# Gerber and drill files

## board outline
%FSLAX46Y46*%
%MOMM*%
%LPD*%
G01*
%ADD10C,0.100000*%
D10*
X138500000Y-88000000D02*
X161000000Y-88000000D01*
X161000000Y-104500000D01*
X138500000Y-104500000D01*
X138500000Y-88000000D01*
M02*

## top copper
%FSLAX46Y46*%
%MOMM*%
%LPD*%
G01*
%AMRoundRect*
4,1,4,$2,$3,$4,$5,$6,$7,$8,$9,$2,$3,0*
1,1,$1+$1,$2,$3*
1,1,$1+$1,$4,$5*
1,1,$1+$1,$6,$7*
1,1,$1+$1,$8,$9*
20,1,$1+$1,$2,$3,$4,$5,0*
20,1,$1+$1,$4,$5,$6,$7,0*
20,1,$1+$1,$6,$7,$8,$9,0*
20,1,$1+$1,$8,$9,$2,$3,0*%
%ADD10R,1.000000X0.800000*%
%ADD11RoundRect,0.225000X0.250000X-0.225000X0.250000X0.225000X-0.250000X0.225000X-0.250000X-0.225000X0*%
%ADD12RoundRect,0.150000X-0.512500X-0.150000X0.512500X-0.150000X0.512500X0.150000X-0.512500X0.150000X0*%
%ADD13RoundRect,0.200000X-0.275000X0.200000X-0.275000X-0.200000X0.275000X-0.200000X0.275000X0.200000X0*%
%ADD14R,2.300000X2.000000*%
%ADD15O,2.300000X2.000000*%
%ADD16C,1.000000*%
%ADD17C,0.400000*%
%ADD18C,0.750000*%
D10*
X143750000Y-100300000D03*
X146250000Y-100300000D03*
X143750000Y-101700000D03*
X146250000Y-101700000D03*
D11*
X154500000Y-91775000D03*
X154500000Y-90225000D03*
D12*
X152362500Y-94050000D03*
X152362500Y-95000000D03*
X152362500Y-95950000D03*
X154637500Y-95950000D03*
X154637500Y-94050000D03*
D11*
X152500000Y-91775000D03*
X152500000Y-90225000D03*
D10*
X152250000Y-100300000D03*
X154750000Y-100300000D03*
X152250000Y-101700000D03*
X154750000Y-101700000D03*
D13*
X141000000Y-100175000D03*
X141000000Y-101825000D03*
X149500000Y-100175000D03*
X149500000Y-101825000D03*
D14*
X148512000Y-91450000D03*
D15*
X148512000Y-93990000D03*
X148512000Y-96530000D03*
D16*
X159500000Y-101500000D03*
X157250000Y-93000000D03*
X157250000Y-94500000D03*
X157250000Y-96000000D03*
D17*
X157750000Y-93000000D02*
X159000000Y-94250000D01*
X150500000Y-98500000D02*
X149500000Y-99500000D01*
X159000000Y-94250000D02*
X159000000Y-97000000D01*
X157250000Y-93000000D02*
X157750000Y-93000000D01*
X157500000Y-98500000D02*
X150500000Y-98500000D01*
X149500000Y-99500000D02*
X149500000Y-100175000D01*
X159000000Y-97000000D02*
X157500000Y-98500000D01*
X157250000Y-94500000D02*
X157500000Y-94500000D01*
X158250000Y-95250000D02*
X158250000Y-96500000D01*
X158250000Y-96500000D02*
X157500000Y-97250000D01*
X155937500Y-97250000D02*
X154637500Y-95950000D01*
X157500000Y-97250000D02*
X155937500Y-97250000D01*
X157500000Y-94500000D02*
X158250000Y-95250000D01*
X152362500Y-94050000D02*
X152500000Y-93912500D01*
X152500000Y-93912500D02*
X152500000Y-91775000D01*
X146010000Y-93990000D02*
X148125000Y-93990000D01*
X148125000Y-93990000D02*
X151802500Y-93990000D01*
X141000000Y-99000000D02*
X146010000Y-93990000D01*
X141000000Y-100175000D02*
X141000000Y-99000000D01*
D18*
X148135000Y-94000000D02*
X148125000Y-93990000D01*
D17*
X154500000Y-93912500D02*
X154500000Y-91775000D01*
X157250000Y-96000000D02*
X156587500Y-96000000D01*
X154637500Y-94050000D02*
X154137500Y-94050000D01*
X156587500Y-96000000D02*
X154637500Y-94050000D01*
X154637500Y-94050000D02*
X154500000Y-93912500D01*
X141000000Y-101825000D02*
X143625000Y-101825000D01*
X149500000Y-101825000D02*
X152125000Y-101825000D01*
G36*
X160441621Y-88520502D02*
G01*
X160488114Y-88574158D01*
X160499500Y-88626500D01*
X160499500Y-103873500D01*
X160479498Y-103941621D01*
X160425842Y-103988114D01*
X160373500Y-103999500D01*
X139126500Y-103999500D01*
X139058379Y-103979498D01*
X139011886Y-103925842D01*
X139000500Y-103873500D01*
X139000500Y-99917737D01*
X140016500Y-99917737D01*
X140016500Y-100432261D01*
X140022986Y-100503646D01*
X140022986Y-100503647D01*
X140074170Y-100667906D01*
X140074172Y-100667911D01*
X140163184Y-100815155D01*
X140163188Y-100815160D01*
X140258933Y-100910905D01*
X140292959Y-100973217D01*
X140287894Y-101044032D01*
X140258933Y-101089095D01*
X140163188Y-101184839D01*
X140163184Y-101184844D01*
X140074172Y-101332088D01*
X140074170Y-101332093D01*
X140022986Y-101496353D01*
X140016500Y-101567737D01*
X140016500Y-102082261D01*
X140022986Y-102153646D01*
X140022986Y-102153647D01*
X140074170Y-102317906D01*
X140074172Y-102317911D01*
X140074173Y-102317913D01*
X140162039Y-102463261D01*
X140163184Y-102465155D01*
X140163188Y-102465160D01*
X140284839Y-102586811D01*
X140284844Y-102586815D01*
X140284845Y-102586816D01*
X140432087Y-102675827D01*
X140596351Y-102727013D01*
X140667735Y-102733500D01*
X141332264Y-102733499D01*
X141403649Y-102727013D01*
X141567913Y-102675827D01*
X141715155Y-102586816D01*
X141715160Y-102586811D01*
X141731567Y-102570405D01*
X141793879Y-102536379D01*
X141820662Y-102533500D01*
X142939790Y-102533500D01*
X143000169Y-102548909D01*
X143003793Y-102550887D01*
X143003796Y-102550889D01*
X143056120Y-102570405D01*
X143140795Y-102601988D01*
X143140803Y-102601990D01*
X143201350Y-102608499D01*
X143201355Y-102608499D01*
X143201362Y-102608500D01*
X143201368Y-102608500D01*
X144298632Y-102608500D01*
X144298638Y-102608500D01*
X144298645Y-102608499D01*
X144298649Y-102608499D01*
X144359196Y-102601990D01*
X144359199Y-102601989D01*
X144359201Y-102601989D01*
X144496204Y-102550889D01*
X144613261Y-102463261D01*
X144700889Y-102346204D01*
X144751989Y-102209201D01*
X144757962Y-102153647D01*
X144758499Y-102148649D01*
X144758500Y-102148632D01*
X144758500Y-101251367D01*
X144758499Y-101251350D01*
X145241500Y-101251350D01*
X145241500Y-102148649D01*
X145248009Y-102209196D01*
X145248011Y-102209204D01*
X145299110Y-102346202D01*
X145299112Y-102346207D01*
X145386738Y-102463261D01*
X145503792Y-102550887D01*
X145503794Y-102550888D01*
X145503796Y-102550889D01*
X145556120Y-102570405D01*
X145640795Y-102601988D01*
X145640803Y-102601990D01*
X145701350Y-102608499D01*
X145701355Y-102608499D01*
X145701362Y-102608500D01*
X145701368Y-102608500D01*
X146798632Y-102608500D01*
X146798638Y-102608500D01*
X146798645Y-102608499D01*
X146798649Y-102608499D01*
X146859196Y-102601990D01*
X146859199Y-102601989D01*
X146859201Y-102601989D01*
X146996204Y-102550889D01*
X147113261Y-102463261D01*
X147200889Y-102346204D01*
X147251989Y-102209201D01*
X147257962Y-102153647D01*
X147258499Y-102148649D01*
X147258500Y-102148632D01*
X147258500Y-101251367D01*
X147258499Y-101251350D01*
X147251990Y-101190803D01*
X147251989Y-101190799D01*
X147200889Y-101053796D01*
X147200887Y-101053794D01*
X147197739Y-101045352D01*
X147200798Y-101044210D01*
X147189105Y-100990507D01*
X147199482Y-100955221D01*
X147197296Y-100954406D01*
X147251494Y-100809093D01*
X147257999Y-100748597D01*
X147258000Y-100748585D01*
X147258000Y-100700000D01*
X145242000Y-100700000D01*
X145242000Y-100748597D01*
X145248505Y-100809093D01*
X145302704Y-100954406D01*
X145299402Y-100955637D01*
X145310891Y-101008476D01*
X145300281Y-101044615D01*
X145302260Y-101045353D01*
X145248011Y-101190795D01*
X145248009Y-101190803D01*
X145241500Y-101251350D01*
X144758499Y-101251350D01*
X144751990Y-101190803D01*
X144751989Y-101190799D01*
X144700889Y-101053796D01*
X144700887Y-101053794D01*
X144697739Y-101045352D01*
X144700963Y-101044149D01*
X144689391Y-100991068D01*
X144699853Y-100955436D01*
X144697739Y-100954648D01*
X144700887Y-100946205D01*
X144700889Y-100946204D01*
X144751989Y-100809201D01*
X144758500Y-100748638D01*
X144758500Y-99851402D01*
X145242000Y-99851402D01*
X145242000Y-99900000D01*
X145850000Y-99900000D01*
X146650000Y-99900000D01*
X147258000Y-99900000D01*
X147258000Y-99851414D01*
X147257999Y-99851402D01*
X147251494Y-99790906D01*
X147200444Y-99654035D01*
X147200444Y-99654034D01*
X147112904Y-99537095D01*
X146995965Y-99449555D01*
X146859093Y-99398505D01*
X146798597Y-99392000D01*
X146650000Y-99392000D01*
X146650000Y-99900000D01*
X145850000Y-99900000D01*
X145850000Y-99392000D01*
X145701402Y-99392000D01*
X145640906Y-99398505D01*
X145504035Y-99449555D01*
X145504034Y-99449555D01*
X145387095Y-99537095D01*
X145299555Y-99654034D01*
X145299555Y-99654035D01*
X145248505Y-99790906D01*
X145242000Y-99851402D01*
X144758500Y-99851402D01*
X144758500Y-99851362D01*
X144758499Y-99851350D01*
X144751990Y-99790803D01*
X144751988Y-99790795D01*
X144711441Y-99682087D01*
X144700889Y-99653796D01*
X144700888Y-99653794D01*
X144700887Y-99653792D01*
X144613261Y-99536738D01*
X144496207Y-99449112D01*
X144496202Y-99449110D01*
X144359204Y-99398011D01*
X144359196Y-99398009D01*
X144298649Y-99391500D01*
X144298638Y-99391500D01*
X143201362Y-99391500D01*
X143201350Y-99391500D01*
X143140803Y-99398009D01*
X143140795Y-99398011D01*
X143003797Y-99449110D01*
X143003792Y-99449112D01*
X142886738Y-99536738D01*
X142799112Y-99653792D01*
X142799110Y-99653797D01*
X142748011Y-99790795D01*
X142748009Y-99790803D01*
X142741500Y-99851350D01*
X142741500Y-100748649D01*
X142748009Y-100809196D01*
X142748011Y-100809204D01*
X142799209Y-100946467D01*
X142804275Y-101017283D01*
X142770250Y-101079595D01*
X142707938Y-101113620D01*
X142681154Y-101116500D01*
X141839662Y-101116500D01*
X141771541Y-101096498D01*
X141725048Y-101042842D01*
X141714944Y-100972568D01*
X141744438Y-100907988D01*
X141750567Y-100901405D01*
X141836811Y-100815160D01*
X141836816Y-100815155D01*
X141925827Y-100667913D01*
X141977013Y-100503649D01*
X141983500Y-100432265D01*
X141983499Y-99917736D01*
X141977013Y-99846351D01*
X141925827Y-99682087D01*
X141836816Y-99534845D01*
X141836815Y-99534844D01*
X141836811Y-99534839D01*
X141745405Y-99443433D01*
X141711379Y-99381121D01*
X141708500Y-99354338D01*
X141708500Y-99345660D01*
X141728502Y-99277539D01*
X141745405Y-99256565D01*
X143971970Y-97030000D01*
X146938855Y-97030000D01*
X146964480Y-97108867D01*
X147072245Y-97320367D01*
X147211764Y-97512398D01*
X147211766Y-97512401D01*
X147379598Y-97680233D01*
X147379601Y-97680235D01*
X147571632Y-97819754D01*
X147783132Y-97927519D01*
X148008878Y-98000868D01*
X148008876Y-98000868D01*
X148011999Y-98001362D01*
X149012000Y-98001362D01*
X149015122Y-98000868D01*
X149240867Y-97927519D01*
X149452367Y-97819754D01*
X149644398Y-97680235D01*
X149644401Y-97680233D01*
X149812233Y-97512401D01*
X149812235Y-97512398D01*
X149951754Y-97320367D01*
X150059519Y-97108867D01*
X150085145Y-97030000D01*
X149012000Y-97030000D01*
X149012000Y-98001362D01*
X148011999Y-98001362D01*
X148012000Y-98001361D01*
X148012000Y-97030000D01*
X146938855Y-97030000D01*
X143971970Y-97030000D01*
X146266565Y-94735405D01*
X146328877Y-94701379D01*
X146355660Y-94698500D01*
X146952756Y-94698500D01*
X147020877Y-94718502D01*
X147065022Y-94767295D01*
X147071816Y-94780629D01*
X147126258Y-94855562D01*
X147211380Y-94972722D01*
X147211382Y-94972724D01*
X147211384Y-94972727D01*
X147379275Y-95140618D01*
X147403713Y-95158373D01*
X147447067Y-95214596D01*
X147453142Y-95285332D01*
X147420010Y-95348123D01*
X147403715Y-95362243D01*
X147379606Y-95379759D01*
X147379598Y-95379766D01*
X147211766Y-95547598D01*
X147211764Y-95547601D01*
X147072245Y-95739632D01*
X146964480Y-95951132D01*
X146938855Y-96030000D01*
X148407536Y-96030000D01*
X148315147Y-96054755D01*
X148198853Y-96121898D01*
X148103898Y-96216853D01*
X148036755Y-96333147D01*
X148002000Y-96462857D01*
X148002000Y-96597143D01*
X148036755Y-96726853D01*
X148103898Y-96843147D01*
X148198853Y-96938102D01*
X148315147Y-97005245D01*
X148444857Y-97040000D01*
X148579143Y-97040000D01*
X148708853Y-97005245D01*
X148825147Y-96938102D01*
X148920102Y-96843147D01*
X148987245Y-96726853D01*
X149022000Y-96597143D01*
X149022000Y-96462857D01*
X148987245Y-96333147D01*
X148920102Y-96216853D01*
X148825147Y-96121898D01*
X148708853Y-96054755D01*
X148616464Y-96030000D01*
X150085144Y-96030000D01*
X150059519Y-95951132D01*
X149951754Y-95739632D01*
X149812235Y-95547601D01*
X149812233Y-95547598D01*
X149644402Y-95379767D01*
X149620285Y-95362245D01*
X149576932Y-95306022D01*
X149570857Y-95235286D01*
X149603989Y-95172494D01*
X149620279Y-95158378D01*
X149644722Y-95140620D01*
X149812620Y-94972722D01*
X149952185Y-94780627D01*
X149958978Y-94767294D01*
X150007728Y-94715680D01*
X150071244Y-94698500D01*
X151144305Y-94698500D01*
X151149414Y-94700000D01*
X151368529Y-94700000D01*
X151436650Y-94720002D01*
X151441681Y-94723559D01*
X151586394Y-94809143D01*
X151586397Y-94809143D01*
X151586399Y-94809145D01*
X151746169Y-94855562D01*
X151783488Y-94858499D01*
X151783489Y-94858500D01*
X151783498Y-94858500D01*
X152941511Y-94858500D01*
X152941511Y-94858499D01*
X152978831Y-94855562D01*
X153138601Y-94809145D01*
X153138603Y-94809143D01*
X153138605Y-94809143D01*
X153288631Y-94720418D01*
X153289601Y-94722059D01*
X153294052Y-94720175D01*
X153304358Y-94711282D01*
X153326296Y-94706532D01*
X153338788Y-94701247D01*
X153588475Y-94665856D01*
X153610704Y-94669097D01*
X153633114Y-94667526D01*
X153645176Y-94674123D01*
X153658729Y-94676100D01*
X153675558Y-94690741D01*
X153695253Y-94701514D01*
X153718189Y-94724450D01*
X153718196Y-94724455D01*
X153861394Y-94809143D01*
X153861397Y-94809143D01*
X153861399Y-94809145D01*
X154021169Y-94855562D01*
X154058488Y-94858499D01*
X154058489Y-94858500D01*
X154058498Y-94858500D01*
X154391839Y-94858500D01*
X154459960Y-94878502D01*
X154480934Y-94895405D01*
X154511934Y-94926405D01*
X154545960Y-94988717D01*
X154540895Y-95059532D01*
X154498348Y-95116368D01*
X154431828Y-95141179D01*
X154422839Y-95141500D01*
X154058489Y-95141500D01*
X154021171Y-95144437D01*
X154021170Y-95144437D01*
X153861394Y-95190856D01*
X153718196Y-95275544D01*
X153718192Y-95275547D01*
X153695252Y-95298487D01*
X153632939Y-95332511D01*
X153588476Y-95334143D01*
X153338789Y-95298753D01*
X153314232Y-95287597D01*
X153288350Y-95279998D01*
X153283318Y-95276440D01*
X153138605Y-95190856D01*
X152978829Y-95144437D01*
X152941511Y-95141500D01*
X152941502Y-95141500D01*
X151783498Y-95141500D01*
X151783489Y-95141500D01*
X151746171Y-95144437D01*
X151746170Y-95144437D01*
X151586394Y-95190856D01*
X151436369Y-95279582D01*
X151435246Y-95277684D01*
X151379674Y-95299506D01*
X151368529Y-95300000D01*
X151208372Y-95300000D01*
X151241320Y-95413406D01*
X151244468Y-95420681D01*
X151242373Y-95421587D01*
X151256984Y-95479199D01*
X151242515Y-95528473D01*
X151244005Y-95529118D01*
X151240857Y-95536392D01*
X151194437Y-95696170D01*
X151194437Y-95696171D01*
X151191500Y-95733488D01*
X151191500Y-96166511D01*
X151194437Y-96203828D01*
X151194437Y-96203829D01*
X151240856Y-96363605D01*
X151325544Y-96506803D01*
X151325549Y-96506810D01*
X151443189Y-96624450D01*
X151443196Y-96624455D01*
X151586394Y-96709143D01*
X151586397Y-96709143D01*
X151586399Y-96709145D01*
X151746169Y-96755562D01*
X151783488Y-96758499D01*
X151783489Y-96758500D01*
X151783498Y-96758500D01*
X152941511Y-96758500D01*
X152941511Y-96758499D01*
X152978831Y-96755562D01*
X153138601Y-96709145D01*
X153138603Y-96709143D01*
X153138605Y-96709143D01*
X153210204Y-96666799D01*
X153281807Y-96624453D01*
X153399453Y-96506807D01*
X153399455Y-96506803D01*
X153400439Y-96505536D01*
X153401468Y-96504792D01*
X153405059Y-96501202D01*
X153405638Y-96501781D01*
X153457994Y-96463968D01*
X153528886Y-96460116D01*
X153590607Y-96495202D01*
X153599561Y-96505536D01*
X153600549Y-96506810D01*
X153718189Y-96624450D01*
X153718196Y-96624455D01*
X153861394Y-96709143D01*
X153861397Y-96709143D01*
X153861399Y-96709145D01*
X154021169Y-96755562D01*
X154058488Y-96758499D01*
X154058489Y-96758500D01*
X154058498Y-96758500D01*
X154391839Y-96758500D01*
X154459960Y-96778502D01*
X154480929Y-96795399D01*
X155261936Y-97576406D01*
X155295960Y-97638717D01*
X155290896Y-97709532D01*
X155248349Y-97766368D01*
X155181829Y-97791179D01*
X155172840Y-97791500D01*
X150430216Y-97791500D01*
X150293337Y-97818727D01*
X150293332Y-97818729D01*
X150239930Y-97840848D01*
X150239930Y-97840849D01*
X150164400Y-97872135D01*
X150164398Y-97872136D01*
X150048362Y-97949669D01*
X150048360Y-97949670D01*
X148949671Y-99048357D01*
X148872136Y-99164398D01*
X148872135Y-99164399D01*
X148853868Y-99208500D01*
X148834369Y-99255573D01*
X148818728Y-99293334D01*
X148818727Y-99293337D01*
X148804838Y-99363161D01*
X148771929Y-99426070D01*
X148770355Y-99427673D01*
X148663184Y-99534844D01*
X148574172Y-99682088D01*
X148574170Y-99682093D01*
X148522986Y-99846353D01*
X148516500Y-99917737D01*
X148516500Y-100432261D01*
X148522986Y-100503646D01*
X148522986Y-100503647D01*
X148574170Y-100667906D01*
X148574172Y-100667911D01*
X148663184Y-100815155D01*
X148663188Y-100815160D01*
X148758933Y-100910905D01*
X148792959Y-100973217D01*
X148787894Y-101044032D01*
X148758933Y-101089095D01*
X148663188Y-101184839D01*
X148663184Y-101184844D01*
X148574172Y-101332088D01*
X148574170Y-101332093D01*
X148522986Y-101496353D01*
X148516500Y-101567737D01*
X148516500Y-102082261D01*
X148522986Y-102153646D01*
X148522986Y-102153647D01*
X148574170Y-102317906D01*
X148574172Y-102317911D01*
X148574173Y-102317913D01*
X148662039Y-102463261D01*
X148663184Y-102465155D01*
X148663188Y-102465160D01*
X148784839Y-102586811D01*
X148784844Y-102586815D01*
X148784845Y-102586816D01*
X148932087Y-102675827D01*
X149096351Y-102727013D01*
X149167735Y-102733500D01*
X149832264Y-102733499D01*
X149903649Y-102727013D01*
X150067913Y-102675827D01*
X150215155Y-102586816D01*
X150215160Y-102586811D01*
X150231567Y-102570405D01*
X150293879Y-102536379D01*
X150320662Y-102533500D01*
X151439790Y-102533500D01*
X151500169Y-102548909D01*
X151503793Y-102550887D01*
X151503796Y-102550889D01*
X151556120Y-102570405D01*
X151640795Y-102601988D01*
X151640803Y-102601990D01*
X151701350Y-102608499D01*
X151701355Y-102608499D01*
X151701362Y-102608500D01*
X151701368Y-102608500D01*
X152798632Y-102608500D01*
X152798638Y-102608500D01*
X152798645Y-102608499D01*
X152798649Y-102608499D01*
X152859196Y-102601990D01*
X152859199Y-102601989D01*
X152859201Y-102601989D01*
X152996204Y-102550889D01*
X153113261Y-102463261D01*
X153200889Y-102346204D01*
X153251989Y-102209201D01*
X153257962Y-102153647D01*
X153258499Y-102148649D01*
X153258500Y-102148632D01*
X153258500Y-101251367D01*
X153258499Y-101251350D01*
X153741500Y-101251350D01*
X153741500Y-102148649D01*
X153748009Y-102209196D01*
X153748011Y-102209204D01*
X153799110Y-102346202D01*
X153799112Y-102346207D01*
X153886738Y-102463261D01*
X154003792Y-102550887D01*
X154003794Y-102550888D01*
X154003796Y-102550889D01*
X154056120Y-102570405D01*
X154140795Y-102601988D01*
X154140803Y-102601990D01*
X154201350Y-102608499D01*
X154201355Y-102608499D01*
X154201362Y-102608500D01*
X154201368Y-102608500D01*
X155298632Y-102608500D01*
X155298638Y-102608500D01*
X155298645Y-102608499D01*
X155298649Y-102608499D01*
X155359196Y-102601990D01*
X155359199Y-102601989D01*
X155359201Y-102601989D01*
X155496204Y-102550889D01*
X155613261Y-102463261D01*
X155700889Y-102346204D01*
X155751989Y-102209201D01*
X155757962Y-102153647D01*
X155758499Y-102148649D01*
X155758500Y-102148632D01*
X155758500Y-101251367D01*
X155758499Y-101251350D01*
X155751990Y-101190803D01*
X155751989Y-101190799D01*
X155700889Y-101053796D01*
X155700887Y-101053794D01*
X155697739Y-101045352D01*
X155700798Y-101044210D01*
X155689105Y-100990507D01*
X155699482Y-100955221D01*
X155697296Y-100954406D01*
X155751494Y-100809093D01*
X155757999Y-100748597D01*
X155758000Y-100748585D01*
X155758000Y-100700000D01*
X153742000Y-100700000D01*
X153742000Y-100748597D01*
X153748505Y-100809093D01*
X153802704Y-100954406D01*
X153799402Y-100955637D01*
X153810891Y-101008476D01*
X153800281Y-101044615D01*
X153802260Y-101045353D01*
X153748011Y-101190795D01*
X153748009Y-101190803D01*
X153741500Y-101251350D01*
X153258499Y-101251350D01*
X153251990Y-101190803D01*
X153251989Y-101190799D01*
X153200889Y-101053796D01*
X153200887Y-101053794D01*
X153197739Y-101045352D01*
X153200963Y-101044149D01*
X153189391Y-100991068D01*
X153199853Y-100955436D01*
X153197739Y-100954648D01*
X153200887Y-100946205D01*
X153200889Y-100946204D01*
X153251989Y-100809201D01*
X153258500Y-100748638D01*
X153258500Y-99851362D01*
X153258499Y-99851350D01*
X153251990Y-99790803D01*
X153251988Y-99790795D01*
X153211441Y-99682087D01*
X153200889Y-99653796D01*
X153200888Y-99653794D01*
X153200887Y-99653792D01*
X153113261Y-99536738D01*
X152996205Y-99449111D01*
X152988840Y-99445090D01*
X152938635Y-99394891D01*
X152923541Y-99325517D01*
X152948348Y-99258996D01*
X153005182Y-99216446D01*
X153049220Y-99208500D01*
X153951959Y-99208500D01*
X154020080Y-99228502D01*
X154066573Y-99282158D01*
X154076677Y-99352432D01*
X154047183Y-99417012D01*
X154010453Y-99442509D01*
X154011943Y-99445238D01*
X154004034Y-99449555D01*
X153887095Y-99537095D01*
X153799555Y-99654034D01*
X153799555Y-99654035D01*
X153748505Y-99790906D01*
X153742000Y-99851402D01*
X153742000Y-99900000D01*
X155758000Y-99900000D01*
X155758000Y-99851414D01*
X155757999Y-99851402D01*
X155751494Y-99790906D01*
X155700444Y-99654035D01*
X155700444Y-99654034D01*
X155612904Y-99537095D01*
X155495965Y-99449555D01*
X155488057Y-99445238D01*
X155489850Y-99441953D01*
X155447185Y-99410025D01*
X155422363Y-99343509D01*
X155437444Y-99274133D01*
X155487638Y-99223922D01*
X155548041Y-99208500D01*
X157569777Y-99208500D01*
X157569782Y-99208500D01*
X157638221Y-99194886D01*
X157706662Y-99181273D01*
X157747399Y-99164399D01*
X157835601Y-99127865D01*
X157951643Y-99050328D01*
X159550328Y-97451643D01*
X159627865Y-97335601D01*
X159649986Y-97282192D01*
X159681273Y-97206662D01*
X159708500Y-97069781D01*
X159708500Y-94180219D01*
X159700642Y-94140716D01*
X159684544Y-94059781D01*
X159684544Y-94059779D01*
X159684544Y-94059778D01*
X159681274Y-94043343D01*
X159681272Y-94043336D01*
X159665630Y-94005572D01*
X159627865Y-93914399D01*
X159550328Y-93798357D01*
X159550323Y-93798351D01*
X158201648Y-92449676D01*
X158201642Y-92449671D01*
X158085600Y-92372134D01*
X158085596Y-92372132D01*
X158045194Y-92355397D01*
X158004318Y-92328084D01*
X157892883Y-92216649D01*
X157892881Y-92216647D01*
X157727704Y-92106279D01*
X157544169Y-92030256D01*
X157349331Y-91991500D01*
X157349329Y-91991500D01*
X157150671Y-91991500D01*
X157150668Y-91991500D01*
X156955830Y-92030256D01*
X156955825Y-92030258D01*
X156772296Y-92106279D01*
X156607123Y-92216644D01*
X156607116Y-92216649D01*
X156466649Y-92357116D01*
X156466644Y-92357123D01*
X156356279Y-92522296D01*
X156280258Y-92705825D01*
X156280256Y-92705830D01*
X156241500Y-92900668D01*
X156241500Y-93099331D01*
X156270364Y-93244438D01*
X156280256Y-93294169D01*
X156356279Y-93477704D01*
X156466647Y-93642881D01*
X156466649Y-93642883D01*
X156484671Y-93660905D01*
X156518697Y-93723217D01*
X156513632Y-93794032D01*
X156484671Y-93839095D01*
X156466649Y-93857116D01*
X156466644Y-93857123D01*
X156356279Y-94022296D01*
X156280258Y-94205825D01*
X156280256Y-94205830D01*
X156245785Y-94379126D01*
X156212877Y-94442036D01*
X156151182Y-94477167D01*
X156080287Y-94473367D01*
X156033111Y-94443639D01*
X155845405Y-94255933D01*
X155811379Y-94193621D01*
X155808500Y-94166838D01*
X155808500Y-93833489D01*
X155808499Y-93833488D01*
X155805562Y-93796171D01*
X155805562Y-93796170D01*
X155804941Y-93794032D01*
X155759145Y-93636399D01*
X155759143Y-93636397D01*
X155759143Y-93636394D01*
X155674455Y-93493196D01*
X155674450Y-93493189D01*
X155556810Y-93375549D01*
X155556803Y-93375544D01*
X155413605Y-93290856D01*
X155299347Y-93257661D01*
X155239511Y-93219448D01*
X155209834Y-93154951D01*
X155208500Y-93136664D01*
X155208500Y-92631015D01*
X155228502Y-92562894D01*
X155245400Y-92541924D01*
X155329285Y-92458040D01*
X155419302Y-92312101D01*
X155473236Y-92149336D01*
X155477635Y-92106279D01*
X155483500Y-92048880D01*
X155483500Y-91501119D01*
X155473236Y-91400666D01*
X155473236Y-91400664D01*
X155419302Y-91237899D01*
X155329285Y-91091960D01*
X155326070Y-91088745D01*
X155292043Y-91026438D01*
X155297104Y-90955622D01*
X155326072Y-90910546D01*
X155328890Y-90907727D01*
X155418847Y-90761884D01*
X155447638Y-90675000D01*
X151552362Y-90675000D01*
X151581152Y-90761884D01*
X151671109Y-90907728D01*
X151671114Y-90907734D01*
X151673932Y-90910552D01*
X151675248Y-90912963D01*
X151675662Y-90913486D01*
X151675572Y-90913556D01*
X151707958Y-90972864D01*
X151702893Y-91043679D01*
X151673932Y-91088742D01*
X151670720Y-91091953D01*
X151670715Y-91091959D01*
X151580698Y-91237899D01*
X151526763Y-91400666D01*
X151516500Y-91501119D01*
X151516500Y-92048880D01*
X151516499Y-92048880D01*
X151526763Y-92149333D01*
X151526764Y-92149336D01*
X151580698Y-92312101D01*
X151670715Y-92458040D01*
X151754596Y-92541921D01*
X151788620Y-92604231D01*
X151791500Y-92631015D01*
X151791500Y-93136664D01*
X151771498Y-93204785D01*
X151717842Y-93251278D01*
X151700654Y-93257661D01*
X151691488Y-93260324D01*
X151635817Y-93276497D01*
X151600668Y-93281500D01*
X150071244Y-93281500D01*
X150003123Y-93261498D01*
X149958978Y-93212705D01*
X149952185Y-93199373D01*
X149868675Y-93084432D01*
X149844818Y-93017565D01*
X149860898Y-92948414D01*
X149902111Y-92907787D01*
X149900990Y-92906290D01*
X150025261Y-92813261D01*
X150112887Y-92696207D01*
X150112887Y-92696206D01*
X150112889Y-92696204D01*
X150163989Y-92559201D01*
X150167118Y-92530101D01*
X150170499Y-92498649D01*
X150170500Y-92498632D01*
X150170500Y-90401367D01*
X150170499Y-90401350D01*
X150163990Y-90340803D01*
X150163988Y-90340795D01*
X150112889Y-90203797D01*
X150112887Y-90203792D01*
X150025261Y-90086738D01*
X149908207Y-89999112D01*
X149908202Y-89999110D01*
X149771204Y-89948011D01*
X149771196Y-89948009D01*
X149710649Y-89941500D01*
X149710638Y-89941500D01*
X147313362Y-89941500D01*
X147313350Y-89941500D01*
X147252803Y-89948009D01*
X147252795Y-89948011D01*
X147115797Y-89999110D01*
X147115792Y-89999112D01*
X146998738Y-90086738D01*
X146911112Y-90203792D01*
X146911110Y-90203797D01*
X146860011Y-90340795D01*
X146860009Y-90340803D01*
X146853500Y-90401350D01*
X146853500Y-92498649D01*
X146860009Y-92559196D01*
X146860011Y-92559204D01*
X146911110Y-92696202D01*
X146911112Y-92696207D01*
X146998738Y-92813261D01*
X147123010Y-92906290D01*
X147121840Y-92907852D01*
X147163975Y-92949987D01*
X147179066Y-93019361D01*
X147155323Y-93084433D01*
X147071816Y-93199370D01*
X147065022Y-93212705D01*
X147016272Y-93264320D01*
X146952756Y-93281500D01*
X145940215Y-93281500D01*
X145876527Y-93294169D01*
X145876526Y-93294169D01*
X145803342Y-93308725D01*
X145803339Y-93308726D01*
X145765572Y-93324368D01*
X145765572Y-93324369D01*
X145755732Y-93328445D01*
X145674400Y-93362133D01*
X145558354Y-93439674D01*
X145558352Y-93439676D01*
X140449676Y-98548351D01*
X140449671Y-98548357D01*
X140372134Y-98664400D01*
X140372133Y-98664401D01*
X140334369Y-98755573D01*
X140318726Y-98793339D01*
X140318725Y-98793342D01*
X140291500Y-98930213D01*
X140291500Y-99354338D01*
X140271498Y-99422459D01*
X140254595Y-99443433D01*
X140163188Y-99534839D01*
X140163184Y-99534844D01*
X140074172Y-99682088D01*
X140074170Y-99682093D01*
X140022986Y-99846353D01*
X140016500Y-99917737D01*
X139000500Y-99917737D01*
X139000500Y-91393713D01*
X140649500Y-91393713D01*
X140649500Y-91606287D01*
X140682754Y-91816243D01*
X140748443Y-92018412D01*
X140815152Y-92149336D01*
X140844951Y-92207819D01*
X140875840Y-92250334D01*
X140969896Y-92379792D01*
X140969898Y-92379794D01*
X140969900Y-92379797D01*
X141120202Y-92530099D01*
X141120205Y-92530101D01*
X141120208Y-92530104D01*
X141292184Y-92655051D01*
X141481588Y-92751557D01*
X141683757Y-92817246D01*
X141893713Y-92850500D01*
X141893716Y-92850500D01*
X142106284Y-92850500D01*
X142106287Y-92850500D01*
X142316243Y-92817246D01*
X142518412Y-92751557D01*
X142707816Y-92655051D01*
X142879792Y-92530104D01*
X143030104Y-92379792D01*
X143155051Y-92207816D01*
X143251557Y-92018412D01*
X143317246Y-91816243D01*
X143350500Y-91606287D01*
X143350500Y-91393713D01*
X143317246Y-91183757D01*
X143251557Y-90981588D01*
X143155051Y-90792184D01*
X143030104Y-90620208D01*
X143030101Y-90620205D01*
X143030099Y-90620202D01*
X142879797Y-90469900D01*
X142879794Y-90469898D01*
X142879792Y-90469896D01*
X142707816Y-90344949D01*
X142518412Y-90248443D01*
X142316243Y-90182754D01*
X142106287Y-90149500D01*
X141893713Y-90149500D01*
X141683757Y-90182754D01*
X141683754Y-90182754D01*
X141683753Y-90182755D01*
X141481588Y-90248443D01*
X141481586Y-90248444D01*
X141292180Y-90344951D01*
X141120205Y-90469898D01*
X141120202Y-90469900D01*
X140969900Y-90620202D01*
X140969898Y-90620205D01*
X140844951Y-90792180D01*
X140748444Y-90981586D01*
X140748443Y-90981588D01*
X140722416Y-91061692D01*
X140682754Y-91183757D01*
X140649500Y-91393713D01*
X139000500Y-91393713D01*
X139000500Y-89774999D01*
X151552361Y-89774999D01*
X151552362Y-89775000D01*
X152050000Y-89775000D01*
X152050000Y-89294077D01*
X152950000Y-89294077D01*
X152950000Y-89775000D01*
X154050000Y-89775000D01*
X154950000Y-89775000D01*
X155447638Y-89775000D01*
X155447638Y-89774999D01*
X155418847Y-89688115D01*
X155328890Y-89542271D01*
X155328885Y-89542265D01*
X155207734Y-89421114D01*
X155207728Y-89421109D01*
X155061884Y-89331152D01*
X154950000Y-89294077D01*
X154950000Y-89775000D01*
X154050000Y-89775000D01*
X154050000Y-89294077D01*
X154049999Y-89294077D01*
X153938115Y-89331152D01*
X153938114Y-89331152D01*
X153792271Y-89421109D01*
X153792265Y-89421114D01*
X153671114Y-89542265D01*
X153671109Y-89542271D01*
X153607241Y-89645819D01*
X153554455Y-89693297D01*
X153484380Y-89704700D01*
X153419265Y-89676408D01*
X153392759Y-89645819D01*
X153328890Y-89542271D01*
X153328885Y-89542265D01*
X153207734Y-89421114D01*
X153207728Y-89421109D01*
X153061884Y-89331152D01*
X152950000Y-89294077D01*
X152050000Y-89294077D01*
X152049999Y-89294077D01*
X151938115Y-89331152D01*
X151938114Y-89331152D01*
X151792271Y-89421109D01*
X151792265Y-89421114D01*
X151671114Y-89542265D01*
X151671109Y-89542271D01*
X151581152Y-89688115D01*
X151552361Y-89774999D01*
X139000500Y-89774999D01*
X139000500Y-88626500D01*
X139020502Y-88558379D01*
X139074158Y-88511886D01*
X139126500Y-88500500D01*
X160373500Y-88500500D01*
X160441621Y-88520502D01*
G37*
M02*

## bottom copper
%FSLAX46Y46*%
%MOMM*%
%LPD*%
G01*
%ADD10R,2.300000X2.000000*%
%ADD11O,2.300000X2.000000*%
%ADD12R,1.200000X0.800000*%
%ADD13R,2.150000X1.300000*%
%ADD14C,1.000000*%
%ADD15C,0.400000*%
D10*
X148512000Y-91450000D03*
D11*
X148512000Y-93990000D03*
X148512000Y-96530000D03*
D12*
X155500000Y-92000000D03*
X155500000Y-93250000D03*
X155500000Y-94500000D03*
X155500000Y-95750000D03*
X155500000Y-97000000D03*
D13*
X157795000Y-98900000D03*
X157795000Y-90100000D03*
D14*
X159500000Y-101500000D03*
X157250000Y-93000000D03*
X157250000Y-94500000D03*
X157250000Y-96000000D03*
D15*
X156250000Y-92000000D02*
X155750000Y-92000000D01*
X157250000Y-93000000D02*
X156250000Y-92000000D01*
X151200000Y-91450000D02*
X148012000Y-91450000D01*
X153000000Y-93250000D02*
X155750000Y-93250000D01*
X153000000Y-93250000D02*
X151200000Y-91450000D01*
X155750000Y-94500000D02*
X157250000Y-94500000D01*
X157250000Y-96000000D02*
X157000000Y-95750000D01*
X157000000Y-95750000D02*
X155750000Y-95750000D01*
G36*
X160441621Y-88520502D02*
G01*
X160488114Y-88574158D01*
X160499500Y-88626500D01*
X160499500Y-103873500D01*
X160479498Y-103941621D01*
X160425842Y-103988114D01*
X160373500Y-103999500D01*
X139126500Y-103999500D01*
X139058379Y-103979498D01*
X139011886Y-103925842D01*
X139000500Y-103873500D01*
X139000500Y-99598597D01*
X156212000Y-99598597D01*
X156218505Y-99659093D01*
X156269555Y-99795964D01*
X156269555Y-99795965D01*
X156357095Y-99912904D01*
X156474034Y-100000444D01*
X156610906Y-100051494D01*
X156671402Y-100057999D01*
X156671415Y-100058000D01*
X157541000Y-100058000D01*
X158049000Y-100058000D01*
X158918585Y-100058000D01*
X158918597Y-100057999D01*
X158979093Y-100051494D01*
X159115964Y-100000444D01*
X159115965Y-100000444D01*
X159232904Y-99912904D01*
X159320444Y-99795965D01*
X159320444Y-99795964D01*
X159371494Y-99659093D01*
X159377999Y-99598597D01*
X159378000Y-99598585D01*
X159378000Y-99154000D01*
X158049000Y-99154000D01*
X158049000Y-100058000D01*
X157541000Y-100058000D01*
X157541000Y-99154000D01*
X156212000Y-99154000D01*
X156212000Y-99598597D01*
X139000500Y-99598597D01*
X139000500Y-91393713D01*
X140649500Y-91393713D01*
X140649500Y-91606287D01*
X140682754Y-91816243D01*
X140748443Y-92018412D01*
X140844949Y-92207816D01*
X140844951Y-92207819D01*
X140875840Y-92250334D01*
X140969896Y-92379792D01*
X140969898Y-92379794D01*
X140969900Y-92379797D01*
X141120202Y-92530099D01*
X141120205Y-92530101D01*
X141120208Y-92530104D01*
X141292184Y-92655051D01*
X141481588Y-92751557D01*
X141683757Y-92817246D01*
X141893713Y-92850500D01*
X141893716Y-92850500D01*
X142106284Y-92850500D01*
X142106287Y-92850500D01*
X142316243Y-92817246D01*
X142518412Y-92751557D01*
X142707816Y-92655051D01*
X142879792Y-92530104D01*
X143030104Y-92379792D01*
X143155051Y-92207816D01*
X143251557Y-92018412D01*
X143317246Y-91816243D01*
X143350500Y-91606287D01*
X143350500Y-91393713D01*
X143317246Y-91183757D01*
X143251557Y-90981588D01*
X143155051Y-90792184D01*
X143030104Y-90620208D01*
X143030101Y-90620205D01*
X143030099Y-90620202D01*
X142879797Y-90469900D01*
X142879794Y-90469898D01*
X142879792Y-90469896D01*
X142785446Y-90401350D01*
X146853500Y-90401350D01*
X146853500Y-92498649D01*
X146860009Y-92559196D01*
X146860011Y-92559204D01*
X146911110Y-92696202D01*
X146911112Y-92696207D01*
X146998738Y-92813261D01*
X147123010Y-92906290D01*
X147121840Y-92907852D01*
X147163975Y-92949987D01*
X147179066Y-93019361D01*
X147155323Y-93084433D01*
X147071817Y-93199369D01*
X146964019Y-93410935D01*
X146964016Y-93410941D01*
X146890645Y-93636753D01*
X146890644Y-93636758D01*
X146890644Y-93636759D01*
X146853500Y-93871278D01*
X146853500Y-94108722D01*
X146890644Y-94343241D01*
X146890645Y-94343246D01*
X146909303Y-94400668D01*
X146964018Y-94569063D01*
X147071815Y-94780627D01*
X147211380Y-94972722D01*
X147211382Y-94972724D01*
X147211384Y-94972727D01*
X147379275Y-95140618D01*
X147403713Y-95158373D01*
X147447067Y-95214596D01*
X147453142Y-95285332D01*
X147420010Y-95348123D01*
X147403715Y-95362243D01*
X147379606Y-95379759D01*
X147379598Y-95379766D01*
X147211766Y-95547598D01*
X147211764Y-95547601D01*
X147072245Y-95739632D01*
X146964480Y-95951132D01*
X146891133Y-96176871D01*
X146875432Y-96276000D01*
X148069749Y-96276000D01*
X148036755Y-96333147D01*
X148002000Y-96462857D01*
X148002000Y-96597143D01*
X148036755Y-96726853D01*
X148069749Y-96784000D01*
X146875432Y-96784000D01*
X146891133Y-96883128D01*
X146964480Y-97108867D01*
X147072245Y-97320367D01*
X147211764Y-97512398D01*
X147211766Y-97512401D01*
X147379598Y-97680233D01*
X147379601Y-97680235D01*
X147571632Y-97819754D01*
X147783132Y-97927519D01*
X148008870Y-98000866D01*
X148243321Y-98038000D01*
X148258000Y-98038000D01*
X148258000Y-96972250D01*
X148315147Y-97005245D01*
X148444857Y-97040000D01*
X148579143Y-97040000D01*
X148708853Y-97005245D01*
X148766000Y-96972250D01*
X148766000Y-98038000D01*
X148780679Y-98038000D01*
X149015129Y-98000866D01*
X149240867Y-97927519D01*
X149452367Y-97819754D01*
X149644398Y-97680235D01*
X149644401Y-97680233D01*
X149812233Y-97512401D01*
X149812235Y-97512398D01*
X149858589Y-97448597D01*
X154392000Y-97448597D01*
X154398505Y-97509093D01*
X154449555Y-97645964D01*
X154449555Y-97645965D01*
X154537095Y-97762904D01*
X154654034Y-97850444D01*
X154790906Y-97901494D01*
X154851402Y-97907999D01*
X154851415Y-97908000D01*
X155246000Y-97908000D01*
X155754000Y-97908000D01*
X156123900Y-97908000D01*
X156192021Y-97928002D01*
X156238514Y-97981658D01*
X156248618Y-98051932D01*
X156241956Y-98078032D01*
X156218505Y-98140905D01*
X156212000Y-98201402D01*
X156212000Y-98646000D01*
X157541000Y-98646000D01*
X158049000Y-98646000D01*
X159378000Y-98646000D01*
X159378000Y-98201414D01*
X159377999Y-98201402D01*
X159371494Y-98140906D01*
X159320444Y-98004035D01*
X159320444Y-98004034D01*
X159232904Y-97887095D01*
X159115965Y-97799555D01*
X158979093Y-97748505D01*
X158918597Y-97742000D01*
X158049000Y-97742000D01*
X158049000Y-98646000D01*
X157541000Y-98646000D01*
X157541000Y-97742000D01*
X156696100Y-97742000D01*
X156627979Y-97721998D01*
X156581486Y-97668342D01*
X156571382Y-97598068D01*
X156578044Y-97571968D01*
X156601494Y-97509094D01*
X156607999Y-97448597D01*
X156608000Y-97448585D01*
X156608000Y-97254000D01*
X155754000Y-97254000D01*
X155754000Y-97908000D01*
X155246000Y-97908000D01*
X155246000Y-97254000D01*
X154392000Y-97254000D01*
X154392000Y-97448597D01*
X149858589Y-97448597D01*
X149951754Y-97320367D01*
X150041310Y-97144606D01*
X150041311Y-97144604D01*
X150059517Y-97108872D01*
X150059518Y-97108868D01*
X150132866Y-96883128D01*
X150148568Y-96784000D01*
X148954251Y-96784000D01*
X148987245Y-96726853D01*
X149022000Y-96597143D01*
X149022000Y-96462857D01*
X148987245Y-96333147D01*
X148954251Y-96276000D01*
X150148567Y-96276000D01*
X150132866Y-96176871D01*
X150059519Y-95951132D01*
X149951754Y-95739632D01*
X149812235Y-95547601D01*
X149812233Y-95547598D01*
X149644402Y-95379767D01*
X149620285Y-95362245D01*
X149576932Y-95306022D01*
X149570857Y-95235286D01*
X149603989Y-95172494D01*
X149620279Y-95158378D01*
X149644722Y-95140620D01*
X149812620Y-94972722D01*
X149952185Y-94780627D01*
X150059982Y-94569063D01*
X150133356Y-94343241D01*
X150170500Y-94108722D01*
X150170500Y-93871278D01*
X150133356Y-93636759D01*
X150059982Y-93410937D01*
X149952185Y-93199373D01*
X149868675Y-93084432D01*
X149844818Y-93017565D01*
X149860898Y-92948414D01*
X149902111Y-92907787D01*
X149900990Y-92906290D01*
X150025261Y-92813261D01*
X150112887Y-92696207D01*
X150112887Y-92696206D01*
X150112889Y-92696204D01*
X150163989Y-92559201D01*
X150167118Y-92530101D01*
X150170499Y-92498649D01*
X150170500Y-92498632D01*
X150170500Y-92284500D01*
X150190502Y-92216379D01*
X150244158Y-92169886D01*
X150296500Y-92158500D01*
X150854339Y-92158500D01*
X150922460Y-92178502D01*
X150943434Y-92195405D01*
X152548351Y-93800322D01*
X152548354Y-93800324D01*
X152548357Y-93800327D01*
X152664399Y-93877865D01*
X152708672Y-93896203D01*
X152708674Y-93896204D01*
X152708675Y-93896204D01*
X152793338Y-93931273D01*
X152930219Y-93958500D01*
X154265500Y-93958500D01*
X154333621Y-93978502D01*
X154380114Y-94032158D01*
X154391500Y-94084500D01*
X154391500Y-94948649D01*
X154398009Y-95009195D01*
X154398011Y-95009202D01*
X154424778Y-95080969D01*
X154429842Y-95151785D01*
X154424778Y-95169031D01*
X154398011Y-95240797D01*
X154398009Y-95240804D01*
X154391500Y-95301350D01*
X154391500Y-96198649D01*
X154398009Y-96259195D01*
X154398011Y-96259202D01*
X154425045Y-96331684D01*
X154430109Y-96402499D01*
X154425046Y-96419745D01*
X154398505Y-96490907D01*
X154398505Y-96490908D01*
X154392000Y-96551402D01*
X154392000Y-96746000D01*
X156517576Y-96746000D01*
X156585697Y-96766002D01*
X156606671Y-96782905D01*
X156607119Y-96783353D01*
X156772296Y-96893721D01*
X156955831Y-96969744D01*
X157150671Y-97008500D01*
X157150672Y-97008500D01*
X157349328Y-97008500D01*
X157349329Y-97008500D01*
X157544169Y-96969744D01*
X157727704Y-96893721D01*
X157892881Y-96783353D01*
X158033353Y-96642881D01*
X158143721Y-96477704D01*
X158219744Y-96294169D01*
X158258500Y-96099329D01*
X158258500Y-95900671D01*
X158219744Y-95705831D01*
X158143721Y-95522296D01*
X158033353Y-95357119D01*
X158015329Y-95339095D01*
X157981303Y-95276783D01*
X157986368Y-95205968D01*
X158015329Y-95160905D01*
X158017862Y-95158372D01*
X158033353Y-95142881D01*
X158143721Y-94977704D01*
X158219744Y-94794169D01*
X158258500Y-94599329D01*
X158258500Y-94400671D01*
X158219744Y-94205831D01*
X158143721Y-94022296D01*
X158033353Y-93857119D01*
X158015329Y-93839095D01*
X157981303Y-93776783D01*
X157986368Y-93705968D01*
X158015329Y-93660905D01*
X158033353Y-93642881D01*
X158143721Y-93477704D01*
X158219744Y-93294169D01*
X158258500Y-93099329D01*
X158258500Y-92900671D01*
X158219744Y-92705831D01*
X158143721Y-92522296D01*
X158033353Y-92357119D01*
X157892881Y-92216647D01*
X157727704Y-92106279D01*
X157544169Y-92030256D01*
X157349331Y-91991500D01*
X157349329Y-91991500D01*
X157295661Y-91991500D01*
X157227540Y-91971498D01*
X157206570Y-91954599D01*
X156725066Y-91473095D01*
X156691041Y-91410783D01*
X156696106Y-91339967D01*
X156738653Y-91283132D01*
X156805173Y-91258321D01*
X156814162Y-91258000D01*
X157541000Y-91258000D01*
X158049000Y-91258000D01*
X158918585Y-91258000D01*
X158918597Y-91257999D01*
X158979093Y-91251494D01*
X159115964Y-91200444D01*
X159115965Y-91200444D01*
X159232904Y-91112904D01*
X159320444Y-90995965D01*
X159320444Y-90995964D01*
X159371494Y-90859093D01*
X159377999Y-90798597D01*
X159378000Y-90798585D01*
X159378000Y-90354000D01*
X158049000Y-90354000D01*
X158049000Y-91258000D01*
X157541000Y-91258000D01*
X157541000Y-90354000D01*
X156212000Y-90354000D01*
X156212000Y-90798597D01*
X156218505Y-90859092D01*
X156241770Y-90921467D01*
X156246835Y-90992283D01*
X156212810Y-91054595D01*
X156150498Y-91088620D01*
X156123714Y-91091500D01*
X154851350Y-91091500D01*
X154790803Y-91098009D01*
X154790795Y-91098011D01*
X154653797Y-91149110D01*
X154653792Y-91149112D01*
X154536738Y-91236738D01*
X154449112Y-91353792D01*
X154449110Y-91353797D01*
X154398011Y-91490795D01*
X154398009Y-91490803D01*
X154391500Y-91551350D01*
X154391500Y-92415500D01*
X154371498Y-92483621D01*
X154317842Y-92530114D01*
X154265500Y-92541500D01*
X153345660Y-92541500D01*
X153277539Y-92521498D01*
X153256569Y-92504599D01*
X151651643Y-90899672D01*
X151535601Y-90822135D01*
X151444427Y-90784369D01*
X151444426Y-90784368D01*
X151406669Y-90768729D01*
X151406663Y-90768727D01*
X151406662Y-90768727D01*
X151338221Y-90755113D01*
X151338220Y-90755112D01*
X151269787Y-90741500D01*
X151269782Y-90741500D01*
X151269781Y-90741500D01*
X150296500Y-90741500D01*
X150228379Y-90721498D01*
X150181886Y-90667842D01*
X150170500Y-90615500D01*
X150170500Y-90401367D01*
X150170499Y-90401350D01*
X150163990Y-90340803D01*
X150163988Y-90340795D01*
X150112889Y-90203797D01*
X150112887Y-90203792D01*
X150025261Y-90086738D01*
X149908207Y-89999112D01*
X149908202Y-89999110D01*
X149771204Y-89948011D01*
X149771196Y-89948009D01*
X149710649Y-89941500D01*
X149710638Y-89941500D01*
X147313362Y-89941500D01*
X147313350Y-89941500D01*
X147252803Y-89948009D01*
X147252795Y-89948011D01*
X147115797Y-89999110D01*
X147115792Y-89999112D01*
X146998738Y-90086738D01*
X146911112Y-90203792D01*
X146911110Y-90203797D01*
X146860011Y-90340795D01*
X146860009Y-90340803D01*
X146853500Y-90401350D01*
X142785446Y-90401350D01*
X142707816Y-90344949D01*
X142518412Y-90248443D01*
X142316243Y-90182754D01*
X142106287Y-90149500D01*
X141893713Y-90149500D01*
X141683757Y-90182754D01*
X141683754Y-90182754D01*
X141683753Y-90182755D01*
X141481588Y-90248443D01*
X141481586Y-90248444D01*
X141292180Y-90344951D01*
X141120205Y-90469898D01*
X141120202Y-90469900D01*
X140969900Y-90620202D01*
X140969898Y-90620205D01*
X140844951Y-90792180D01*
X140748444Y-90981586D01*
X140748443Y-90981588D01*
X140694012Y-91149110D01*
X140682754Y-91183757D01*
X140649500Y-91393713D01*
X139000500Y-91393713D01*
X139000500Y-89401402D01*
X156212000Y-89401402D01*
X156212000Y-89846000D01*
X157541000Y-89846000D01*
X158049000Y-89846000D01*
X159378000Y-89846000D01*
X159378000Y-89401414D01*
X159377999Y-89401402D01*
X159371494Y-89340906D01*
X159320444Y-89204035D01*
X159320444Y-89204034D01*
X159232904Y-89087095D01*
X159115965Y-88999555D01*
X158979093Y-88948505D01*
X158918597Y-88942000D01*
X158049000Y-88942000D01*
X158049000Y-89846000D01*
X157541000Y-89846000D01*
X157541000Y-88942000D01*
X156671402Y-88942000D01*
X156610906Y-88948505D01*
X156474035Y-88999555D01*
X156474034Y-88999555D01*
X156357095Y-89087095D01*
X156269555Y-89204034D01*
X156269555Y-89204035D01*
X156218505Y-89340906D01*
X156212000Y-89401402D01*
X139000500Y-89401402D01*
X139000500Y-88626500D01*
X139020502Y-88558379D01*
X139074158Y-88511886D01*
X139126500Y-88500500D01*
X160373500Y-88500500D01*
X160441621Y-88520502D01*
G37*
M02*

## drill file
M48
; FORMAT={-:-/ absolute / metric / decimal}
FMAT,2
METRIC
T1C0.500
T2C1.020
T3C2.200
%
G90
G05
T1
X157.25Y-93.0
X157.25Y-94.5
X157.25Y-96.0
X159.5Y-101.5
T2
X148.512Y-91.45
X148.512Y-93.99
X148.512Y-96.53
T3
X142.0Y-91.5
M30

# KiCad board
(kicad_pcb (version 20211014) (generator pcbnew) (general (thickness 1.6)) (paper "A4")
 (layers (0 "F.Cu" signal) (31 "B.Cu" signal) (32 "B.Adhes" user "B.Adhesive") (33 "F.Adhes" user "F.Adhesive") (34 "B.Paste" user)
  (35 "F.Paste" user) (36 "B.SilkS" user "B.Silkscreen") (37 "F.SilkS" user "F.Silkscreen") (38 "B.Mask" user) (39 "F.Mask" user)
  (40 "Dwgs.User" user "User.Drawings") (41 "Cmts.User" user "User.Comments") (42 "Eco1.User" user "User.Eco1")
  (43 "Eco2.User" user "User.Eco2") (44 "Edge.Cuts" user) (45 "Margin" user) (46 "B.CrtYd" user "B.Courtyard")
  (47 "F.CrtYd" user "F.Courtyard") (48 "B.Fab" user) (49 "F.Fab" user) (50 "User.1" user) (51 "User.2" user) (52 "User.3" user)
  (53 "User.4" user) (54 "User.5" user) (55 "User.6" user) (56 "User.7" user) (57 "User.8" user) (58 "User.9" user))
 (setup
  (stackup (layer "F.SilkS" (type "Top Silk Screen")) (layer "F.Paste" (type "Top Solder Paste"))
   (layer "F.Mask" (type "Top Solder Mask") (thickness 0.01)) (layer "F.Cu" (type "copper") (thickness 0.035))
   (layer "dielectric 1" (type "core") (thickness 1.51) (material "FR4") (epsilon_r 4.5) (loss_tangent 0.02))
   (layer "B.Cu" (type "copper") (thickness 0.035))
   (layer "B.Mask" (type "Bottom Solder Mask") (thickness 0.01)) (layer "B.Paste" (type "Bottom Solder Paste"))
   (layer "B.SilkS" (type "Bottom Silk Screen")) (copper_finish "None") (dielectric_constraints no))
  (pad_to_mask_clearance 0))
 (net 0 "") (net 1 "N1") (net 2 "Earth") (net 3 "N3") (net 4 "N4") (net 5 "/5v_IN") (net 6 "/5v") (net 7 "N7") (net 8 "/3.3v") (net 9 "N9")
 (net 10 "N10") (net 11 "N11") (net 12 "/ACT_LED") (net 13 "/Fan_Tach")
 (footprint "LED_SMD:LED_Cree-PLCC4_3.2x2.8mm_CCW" (layer "F.Cu") (at 145 101)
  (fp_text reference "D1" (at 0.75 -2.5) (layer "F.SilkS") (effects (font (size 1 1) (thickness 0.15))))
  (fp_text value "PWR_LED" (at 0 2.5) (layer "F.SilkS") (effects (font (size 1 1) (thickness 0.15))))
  (pad "0" smd rect (at -1.25 -0.7) (size 1 0.8) (layers "F.Cu" "F.Paste" "F.Mask") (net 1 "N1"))
  (pad "1" smd rect (at 1.25 -0.7) (size 1 0.8) (layers "F.Cu" "F.Paste" "F.Mask") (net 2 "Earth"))
  (pad "2" smd rect (at -1.25 0.7) (size 1 0.8) (layers "F.Cu" "F.Paste" "F.Mask") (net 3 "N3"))
  (pad "3" smd rect (at 1.25 0.7) (size 1 0.8) (layers "F.Cu" "F.Paste" "F.Mask") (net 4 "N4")))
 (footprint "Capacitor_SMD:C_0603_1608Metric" (layer "F.Cu") (at 154.5 91 90)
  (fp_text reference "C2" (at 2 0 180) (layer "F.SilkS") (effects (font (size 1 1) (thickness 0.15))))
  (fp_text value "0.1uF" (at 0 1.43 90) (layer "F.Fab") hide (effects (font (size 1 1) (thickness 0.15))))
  (pad "1" smd roundrect (at -0.775 0 90) (size 0.9 0.95) (layers "F.Cu" "F.Paste" "F.Mask") (roundrect_rratio 0.25) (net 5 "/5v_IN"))
  (pad "2" smd roundrect (at 0.775 0 90) (size 0.9 0.95) (layers "F.Cu" "F.Paste" "F.Mask") (roundrect_rratio 0.25) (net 2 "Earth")))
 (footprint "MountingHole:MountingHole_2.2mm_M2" (layer "F.Cu") (at 142 91.5)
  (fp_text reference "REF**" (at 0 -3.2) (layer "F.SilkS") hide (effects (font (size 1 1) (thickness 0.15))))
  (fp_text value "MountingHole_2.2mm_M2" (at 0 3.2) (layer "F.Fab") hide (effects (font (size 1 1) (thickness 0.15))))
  (pad "" np_thru_hole circle (at 0 0) (size 2.2 2.2) (drill 2.2) (layers *.Cu *.Mask)))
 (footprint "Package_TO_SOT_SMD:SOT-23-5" (layer "F.Cu") (at 153.5 95)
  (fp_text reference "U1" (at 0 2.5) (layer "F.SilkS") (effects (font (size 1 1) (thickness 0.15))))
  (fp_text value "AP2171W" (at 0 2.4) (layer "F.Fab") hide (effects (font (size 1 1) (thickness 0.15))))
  (pad "1" smd roundrect (at -1.1375 -0.95) (size 1.325 0.6) (layers "F.Cu" "F.Paste" "F.Mask") (roundrect_rratio 0.25) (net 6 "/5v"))
  (pad "2" smd roundrect (at -1.1375 0) (size 1.325 0.6) (layers "F.Cu" "F.Paste" "F.Mask") (roundrect_rratio 0.25) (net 2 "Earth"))
  (pad "3" smd roundrect (at -1.1375 0.95) (size 1.325 0.6) (layers "F.Cu" "F.Paste" "F.Mask") (roundrect_rratio 0.25) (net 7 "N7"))
  (pad "4" smd roundrect (at 1.1375 0.95) (size 1.325 0.6) (layers "F.Cu" "F.Paste" "F.Mask") (roundrect_rratio 0.25) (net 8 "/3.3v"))
  (pad "5" smd roundrect (at 1.1375 -0.95) (size 1.325 0.6) (layers "F.Cu" "F.Paste" "F.Mask") (roundrect_rratio 0.25) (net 5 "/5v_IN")))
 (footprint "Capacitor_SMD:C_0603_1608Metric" (layer "F.Cu") (at 152.5 91 90)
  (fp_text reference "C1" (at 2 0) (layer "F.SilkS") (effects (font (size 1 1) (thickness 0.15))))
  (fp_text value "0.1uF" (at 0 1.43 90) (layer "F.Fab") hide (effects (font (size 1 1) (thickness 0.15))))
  (pad "1" smd roundrect (at -0.775 0 90) (size 0.9 0.95) (layers "F.Cu" "F.Paste" "F.Mask") (roundrect_rratio 0.25) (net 6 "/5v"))
  (pad "2" smd roundrect (at 0.775 0 90) (size 0.9 0.95) (layers "F.Cu" "F.Paste" "F.Mask") (roundrect_rratio 0.25) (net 2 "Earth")))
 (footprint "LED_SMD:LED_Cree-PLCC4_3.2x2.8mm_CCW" (layer "F.Cu") (at 153.5 101)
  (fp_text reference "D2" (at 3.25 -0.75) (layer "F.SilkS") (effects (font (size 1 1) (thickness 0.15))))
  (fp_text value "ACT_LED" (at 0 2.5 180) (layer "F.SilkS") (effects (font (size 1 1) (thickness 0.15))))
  (pad "0" smd rect (at -1.25 -0.7) (size 1 0.8) (layers "F.Cu" "F.Paste" "F.Mask") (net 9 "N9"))
  (pad "1" smd rect (at 1.25 -0.7) (size 1 0.8) (layers "F.Cu" "F.Paste" "F.Mask") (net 2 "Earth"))
  (pad "2" smd rect (at -1.25 0.7) (size 1 0.8) (layers "F.Cu" "F.Paste" "F.Mask") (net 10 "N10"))
  (pad "3" smd rect (at 1.25 0.7) (size 1 0.8) (layers "F.Cu" "F.Paste" "F.Mask") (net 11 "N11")))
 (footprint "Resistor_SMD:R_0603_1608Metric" (layer "F.Cu") (at 141 101 -90)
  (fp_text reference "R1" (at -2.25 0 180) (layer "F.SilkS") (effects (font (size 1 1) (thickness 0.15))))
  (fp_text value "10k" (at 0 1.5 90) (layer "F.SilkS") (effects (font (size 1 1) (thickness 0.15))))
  (pad "1" smd roundrect (at -0.825 0 270) (size 0.8 0.95) (layers "F.Cu" "F.Paste" "F.Mask") (roundrect_rratio 0.25) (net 6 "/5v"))
  (pad "2" smd roundrect (at 0.825 0 270) (size 0.8 0.95) (layers "F.Cu" "F.Paste" "F.Mask") (roundrect_rratio 0.25) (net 3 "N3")))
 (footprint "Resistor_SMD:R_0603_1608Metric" (layer "F.Cu") (at 149.5 101 -90)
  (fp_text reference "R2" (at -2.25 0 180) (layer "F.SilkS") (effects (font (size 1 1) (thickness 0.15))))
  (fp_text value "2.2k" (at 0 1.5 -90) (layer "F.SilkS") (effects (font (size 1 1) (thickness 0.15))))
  (pad "1" smd roundrect (at -0.825 0 270) (size 0.8 0.95) (layers "F.Cu" "F.Paste" "F.Mask") (roundrect_rratio 0.25) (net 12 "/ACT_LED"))
  (pad "2" smd roundrect (at 0.825 0 270) (size 0.8 0.95) (layers "F.Cu" "F.Paste" "F.Mask") (roundrect_rratio 0.25) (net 10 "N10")))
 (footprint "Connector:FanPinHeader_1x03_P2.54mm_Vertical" (layer "B.Cu") (at 147.75 91.45 -90)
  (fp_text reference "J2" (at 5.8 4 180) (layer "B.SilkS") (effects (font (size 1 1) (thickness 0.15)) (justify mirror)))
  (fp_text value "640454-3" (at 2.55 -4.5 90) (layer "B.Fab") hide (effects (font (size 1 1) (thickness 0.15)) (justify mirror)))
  (pad "1" thru_hole rect (at 0 -0.762 180) (size 2.3 2) (drill 1.02) (layers *.Cu *.Mask) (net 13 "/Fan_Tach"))
  (pad "2" thru_hole oval (at 2.54 -0.762 180) (size 2.3 2) (drill 1.02) (layers *.Cu *.Mask) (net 6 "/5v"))
  (pad "3" thru_hole oval (at 5.08 -0.762 180) (size 2.3 2) (drill 1.02) (layers *.Cu *.Mask) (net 2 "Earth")))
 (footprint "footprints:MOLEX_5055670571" (layer "B.Cu") (at 157.25 94.5 90)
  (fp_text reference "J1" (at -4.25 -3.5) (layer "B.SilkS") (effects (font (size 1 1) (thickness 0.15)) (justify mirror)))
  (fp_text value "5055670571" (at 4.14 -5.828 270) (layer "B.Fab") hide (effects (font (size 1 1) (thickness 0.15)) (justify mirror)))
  (pad "1" smd rect (at 2.5 -1.75 90) (size 0.8 1.2) (layers "B.Cu" "B.Paste") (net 12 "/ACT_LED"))
  (pad "2" smd rect (at 1.25 -1.75 90) (size 0.8 1.2) (layers "B.Cu" "B.Paste") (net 13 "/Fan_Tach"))
  (pad "3" smd rect (at 0 -1.75 90) (size 0.8 1.2) (layers "B.Cu" "B.Paste") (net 8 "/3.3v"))
  (pad "4" smd rect (at -1.25 -1.75 90) (size 0.8 1.2) (layers "B.Cu" "B.Paste") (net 5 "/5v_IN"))
  (pad "5" smd rect (at -2.5 -1.75 90) (size 0.8 1.2) (layers "B.Cu" "B.Paste") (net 2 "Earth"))
  (pad "S1" smd rect (at -4.4 0.545 90) (size 1.3 2.15) (layers "B.Cu" "B.Paste") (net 2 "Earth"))
  (pad "S2" smd rect (at 4.4 0.545 90) (size 1.3 2.15) (layers "B.Cu" "B.Paste") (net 2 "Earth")))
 (gr_rect (start 138.5 88) (end 161 104.5) (layer "Edge.Cuts") (width 0.1) (fill none))
 (via (at 159.5 101.5) (size 1) (drill 0.5) (layers "F.Cu" "B.Cu") (free) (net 2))
 (segment (start 157.75 93) (end 159 94.25) (width 0.4) (layer "F.Cu") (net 12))
 (segment (start 150.5 98.5) (end 149.5 99.5) (width 0.4) (layer "F.Cu") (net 12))
 (segment (start 159 94.25) (end 159 97) (width 0.4) (layer "F.Cu") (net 12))
 (segment (start 157.25 93) (end 157.75 93) (width 0.4) (layer "F.Cu") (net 12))
 (segment (start 157.5 98.5) (end 150.5 98.5) (width 0.4) (layer "F.Cu") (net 12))
 (segment (start 149.5 99.5) (end 149.5 100.175) (width 0.4) (layer "F.Cu") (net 12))
 (segment (start 159 97) (end 157.5 98.5) (width 0.4) (layer "F.Cu") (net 12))
 (via (at 157.25 93) (size 1) (drill 0.5) (layers "F.Cu" "B.Cu") (free) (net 12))
 (segment (start 156.25 92) (end 155.75 92) (width 0.4) (layer "B.Cu") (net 12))
 (segment (start 157.25 93) (end 156.25 92) (width 0.4) (layer "B.Cu") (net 12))
 (segment (start 151.2 91.45) (end 148.012 91.45) (width 0.4) (layer "B.Cu") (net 13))
 (segment (start 153 93.25) (end 155.75 93.25) (width 0.4) (layer "B.Cu") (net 13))
 (segment (start 153 93.25) (end 151.2 91.45) (width 0.4) (layer "B.Cu") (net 13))
 (segment (start 157.25 94.5) (end 157.5 94.5) (width 0.4) (layer "F.Cu") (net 8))
 (segment (start 158.25 95.25) (end 158.25 96.5) (width 0.4) (layer "F.Cu") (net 8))
 (segment (start 158.25 96.5) (end 157.5 97.25) (width 0.4) (layer "F.Cu") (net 8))
 (segment (start 155.9375 97.25) (end 154.6375 95.95) (width 0.4) (layer "F.Cu") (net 8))
 (segment (start 157.5 97.25) (end 155.9375 97.25) (width 0.4) (layer "F.Cu") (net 8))
 (segment (start 157.5 94.5) (end 158.25 95.25) (width 0.4) (layer "F.Cu") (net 8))
 (via (at 157.25 94.5) (size 1) (drill 0.5) (layers "F.Cu" "B.Cu") (free) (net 8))
 (segment (start 155.75 94.5) (end 157.25 94.5) (width 0.4) (layer "B.Cu") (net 8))
 (segment (start 152.3625 94.05) (end 152.5 93.9125) (width 0.4) (layer "F.Cu") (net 6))
 (segment (start 152.5 93.9125) (end 152.5 91.775) (width 0.4) (layer "F.Cu") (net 6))
 (segment (start 146.01 93.99) (end 148.125 93.99) (width 0.4) (layer "F.Cu") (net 6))
 (segment (start 148.125 93.99) (end 151.8025 93.99) (width 0.4) (layer "F.Cu") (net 6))
 (segment (start 141 99) (end 146.01 93.99) (width 0.4) (layer "F.Cu") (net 6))
 (segment (start 141 100.175) (end 141 99) (width 0.4) (layer "F.Cu") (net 6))
 (segment (start 148.135 94) (end 148.125 93.99) (width 0.75) (layer "F.Cu") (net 6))
 (segment (start 154.5 93.9125) (end 154.5 91.775) (width 0.4) (layer "F.Cu") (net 5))
 (segment (start 157.25 96) (end 156.5875 96) (width 0.4) (layer "F.Cu") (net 5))
 (segment (start 154.6375 94.05) (end 154.1375 94.05) (width 0.4) (layer "F.Cu") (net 5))
 (segment (start 156.5875 96) (end 154.6375 94.05) (width 0.4) (layer "F.Cu") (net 5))
 (segment (start 154.6375 94.05) (end 154.5 93.9125) (width 0.4) (layer "F.Cu") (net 5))
 (via (at 157.25 96) (size 1) (drill 0.5) (layers "F.Cu" "B.Cu") (free) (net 5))
 (segment (start 157.25 96) (end 157 95.75) (width 0.4) (layer "B.Cu") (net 5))
 (segment (start 157 95.75) (end 155.75 95.75) (width 0.4) (layer "B.Cu") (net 5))
 (segment (start 141 101.825) (end 143.625 101.825) (width 0.4) (layer "F.Cu") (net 3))
 (segment (start 149.5 101.825) (end 152.125 101.825) (width 0.4) (layer "F.Cu") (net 10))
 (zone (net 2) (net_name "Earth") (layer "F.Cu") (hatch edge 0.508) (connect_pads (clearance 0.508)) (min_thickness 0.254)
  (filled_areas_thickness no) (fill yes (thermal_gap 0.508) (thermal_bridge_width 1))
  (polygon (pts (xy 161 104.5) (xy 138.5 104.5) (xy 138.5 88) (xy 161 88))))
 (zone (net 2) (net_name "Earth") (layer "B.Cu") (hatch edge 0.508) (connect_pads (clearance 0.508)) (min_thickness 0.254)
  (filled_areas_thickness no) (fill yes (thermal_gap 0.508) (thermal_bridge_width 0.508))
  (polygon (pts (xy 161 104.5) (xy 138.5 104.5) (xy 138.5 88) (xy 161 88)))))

